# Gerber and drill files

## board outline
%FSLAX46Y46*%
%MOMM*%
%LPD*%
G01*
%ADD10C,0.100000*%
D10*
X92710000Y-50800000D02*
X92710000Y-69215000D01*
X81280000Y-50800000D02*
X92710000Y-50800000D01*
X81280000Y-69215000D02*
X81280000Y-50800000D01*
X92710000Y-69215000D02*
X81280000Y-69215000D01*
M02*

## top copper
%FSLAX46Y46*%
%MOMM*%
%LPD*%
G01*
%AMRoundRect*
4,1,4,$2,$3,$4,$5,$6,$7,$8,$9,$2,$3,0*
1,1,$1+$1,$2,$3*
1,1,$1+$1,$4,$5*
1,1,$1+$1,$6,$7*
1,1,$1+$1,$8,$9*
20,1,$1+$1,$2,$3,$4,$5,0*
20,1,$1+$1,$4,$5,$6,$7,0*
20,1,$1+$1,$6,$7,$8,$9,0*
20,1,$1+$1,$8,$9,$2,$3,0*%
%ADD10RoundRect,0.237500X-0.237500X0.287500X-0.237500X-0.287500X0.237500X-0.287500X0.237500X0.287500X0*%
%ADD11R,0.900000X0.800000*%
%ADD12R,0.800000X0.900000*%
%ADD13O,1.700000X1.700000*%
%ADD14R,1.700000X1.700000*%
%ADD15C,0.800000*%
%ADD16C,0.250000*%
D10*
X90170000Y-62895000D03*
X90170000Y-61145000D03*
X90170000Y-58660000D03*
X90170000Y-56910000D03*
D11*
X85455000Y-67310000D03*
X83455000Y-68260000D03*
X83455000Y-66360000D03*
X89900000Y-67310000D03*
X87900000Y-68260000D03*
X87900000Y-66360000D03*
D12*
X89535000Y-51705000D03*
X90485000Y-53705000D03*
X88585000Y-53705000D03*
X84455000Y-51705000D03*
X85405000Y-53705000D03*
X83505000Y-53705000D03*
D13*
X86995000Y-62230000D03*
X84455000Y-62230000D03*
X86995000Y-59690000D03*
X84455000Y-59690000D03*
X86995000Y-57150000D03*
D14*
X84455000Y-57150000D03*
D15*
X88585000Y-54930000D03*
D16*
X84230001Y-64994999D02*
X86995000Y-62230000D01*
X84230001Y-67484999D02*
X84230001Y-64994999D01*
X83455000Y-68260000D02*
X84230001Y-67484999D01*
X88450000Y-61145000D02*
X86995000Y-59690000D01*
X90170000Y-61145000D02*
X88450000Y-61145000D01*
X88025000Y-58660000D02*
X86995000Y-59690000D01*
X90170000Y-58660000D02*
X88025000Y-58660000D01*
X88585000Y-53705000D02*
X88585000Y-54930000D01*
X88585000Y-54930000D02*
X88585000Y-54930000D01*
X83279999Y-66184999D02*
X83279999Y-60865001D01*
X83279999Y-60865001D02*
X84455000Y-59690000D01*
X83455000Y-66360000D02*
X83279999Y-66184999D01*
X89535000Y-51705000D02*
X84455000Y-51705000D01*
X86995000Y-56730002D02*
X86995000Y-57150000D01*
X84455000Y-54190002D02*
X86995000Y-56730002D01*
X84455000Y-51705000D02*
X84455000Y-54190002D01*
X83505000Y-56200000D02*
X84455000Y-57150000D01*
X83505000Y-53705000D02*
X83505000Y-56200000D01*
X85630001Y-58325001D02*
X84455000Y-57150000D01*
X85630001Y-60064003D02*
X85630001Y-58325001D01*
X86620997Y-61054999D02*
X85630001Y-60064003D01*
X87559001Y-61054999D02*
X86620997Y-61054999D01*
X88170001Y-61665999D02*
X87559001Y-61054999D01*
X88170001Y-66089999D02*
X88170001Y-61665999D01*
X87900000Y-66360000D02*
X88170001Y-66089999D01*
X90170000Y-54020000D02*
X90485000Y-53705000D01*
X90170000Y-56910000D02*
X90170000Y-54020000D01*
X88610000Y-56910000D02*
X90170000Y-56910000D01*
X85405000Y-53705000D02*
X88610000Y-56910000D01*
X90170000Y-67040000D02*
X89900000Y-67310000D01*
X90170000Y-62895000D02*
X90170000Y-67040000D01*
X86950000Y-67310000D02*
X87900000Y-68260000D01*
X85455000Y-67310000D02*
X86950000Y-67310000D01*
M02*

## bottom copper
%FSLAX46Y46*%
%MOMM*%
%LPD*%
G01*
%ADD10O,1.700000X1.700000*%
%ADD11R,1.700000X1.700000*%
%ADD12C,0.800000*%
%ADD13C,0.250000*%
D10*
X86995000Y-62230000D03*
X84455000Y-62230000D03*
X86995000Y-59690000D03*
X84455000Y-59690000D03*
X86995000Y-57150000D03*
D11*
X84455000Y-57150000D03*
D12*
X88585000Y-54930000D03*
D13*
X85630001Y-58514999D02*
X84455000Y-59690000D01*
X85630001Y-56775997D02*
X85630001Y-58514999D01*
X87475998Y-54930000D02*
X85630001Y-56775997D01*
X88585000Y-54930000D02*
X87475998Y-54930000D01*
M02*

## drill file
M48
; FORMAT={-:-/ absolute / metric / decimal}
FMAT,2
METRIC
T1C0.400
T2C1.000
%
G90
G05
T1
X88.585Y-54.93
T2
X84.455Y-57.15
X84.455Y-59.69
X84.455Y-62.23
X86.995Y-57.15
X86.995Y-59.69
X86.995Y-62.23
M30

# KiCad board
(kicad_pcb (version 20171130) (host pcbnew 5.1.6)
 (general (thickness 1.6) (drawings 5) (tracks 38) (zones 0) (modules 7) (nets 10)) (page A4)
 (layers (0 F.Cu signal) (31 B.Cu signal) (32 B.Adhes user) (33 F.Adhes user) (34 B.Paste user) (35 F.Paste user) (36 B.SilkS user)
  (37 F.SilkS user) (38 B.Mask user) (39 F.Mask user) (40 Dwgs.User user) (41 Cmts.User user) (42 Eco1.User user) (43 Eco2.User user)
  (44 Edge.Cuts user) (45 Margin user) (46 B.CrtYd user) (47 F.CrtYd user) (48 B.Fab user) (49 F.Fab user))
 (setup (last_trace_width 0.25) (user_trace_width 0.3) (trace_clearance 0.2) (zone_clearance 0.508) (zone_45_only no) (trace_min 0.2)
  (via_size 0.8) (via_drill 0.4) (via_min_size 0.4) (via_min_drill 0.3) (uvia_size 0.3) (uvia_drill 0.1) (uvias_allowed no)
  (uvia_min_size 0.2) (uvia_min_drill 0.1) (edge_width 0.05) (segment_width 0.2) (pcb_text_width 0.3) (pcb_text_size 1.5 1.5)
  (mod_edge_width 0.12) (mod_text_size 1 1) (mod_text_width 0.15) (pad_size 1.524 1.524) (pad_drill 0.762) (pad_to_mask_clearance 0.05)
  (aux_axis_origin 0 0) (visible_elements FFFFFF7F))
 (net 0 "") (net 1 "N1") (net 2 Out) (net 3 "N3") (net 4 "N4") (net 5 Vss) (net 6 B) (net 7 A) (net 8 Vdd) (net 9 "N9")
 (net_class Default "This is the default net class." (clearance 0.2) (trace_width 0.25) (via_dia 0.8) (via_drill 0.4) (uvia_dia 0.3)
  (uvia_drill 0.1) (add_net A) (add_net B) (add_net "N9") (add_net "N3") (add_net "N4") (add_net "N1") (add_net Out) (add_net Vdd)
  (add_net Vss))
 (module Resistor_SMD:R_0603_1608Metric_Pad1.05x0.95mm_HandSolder (layer F.Cu) (at 90.17 62.02 270)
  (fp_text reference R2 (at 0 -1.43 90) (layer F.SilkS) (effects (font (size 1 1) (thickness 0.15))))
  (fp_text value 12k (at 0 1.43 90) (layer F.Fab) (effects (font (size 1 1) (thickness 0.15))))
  (pad 2 smd roundrect (at 0.875 0 270) (size 1.05 0.95) (layers F.Cu F.Paste F.Mask) (roundrect_rratio 0.25) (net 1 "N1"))
  (pad 1 smd roundrect (at -0.875 0 270) (size 1.05 0.95) (layers F.Cu F.Paste F.Mask) (roundrect_rratio 0.25) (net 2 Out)))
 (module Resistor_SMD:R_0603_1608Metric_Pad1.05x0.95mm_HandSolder (layer F.Cu) (at 90.17 57.785 270)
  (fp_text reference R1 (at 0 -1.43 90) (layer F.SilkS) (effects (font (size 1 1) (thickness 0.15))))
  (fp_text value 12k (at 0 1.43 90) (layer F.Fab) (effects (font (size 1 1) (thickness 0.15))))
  (pad 2 smd roundrect (at 0.875 0 270) (size 1.05 0.95) (layers F.Cu F.Paste F.Mask) (roundrect_rratio 0.25) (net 2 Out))
  (pad 1 smd roundrect (at -0.875 0 270) (size 1.05 0.95) (layers F.Cu F.Paste F.Mask) (roundrect_rratio 0.25) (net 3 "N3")))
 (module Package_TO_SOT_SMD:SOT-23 (layer F.Cu) (at 84.455 67.31)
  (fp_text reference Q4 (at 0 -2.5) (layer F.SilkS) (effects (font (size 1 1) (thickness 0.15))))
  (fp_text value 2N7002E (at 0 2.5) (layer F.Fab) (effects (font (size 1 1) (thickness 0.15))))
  (pad 3 smd rect (at 1 0) (size 0.9 0.8) (layers F.Cu F.Paste F.Mask) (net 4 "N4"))
  (pad 2 smd rect (at -1 0.95) (size 0.9 0.8) (layers F.Cu F.Paste F.Mask) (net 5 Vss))
  (pad 1 smd rect (at -1 -0.95) (size 0.9 0.8) (layers F.Cu F.Paste F.Mask) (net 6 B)))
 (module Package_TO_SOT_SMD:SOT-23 (layer F.Cu) (at 88.9 67.31)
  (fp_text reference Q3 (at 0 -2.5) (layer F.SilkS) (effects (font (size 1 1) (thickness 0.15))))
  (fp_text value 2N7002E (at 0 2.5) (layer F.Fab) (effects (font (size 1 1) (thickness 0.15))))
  (pad 3 smd rect (at 1 0) (size 0.9 0.8) (layers F.Cu F.Paste F.Mask) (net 1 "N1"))
  (pad 2 smd rect (at -1 0.95) (size 0.9 0.8) (layers F.Cu F.Paste F.Mask) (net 4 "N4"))
  (pad 1 smd rect (at -1 -0.95) (size 0.9 0.8) (layers F.Cu F.Paste F.Mask) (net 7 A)))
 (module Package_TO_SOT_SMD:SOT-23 (layer F.Cu) (at 89.535 52.705 90)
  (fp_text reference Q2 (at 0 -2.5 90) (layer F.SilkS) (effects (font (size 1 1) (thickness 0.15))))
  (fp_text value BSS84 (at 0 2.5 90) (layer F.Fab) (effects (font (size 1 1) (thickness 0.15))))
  (pad 3 smd rect (at 1 0 90) (size 0.9 0.8) (layers F.Cu F.Paste F.Mask) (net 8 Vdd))
  (pad 2 smd rect (at -1 0.95 90) (size 0.9 0.8) (layers F.Cu F.Paste F.Mask) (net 3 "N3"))
  (pad 1 smd rect (at -1 -0.95 90) (size 0.9 0.8) (layers F.Cu F.Paste F.Mask) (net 6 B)))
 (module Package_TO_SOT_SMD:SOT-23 (layer F.Cu) (at 84.455 52.705 90)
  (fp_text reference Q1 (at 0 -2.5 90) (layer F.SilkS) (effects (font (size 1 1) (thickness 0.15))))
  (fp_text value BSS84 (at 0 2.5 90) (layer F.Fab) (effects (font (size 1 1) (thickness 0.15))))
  (pad 3 smd rect (at 1 0 90) (size 0.9 0.8) (layers F.Cu F.Paste F.Mask) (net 8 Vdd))
  (pad 2 smd rect (at -1 0.95 90) (size 0.9 0.8) (layers F.Cu F.Paste F.Mask) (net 3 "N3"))
  (pad 1 smd rect (at -1 -0.95 90) (size 0.9 0.8) (layers F.Cu F.Paste F.Mask) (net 7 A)))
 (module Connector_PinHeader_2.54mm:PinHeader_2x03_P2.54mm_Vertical (layer F.Cu) (at 84.455 57.15)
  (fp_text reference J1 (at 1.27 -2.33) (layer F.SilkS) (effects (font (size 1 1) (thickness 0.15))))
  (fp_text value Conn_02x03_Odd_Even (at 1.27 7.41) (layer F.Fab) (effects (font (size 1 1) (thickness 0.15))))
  (pad 6 thru_hole oval (at 2.54 5.08) (size 1.7 1.7) (drill 1) (layers *.Cu *.Mask) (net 5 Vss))
  (pad 5 thru_hole oval (at 0 5.08) (size 1.7 1.7) (drill 1) (layers *.Cu *.Mask) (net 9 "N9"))
  (pad 4 thru_hole oval (at 2.54 2.54) (size 1.7 1.7) (drill 1) (layers *.Cu *.Mask) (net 2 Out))
  (pad 3 thru_hole oval (at 0 2.54) (size 1.7 1.7) (drill 1) (layers *.Cu *.Mask) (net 6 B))
  (pad 2 thru_hole oval (at 2.54 0) (size 1.7 1.7) (drill 1) (layers *.Cu *.Mask) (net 8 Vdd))
  (pad 1 thru_hole rect (at 0 0) (size 1.7 1.7) (drill 1) (layers *.Cu *.Mask) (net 7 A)))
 (gr_line (start 92.71 50.8) (end 92.71 69.215) (layer Edge.Cuts) (width 0.1))
 (gr_line (start 81.28 50.8) (end 92.71 50.8) (layer Edge.Cuts) (width 0.1))
 (gr_line (start 81.28 69.215) (end 81.28 50.8) (layer Edge.Cuts) (width 0.1))
 (gr_line (start 92.71 69.215) (end 81.28 69.215) (layer Edge.Cuts) (width 0.1))
 (segment (start 84.230001 64.994999) (end 86.995 62.23) (width 0.25) (layer F.Cu) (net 5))
 (segment (start 84.230001 67.484999) (end 84.230001 64.994999) (width 0.25) (layer F.Cu) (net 5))
 (segment (start 83.455 68.26) (end 84.230001 67.484999) (width 0.25) (layer F.Cu) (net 5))
 (segment (start 88.45 61.145) (end 86.995 59.69) (width 0.25) (layer F.Cu) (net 2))
 (segment (start 90.17 61.145) (end 88.45 61.145) (width 0.25) (layer F.Cu) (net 2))
 (segment (start 88.025 58.66) (end 86.995 59.69) (width 0.25) (layer F.Cu) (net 2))
 (segment (start 90.17 58.66) (end 88.025 58.66) (width 0.25) (layer F.Cu) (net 2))
 (segment (start 88.585 53.705) (end 88.585 54.93) (width 0.25) (layer F.Cu) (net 6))
 (segment (start 88.585 54.93) (end 88.585 54.93) (width 0.25) (layer F.Cu) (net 6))
 (via (at 88.585 54.93) (size 0.8) (drill 0.4) (layers F.Cu B.Cu) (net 6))
 (segment (start 85.630001 58.514999) (end 84.455 59.69) (width 0.25) (layer B.Cu) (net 6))
 (segment (start 85.630001 56.775997) (end 85.630001 58.514999) (width 0.25) (layer B.Cu) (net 6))
 (segment (start 87.475998 54.93) (end 85.630001 56.775997) (width 0.25) (layer B.Cu) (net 6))
 (segment (start 88.585 54.93) (end 87.475998 54.93) (width 0.25) (layer B.Cu) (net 6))
 (segment (start 83.279999 66.184999) (end 83.279999 60.865001) (width 0.25) (layer F.Cu) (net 6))
 (segment (start 83.279999 60.865001) (end 84.455 59.69) (width 0.25) (layer F.Cu) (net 6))
 (segment (start 83.455 66.36) (end 83.279999 66.184999) (width 0.25) (layer F.Cu) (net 6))
 (segment (start 89.535 51.705) (end 84.455 51.705) (width 0.25) (layer F.Cu) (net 8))
 (segment (start 86.995 56.730002) (end 86.995 57.15) (width 0.25) (layer F.Cu) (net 8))
 (segment (start 84.455 54.190002) (end 86.995 56.730002) (width 0.25) (layer F.Cu) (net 8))
 (segment (start 84.455 51.705) (end 84.455 54.190002) (width 0.25) (layer F.Cu) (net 8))
 (segment (start 83.505 56.2) (end 84.455 57.15) (width 0.25) (layer F.Cu) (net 7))
 (segment (start 83.505 53.705) (end 83.505 56.2) (width 0.25) (layer F.Cu) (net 7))
 (segment (start 85.630001 58.325001) (end 84.455 57.15) (width 0.25) (layer F.Cu) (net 7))
 (segment (start 85.630001 60.064003) (end 85.630001 58.325001) (width 0.25) (layer F.Cu) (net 7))
 (segment (start 86.620997 61.054999) (end 85.630001 60.064003) (width 0.25) (layer F.Cu) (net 7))
 (segment (start 87.559001 61.054999) (end 86.620997 61.054999) (width 0.25) (layer F.Cu) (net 7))
 (segment (start 88.170001 61.665999) (end 87.559001 61.054999) (width 0.25) (layer F.Cu) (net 7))
 (segment (start 88.170001 66.089999) (end 88.170001 61.665999) (width 0.25) (layer F.Cu) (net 7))
 (segment (start 87.9 66.36) (end 88.170001 66.089999) (width 0.25) (layer F.Cu) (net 7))
 (segment (start 90.17 54.02) (end 90.485 53.705) (width 0.25) (layer F.Cu) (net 3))
 (segment (start 90.17 56.91) (end 90.17 54.02) (width 0.25) (layer F.Cu) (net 3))
 (segment (start 88.61 56.91) (end 90.17 56.91) (width 0.25) (layer F.Cu) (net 3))
 (segment (start 85.405 53.705) (end 88.61 56.91) (width 0.25) (layer F.Cu) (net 3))
 (segment (start 90.17 67.04) (end 89.9 67.31) (width 0.25) (layer F.Cu) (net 1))
 (segment (start 90.17 62.895) (end 90.17 67.04) (width 0.25) (layer F.Cu) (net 1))
 (segment (start 86.95 67.31) (end 87.9 68.26) (width 0.25) (layer F.Cu) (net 4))
 (segment (start 85.455 67.31) (end 86.95 67.31) (width 0.25) (layer F.Cu) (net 4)))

